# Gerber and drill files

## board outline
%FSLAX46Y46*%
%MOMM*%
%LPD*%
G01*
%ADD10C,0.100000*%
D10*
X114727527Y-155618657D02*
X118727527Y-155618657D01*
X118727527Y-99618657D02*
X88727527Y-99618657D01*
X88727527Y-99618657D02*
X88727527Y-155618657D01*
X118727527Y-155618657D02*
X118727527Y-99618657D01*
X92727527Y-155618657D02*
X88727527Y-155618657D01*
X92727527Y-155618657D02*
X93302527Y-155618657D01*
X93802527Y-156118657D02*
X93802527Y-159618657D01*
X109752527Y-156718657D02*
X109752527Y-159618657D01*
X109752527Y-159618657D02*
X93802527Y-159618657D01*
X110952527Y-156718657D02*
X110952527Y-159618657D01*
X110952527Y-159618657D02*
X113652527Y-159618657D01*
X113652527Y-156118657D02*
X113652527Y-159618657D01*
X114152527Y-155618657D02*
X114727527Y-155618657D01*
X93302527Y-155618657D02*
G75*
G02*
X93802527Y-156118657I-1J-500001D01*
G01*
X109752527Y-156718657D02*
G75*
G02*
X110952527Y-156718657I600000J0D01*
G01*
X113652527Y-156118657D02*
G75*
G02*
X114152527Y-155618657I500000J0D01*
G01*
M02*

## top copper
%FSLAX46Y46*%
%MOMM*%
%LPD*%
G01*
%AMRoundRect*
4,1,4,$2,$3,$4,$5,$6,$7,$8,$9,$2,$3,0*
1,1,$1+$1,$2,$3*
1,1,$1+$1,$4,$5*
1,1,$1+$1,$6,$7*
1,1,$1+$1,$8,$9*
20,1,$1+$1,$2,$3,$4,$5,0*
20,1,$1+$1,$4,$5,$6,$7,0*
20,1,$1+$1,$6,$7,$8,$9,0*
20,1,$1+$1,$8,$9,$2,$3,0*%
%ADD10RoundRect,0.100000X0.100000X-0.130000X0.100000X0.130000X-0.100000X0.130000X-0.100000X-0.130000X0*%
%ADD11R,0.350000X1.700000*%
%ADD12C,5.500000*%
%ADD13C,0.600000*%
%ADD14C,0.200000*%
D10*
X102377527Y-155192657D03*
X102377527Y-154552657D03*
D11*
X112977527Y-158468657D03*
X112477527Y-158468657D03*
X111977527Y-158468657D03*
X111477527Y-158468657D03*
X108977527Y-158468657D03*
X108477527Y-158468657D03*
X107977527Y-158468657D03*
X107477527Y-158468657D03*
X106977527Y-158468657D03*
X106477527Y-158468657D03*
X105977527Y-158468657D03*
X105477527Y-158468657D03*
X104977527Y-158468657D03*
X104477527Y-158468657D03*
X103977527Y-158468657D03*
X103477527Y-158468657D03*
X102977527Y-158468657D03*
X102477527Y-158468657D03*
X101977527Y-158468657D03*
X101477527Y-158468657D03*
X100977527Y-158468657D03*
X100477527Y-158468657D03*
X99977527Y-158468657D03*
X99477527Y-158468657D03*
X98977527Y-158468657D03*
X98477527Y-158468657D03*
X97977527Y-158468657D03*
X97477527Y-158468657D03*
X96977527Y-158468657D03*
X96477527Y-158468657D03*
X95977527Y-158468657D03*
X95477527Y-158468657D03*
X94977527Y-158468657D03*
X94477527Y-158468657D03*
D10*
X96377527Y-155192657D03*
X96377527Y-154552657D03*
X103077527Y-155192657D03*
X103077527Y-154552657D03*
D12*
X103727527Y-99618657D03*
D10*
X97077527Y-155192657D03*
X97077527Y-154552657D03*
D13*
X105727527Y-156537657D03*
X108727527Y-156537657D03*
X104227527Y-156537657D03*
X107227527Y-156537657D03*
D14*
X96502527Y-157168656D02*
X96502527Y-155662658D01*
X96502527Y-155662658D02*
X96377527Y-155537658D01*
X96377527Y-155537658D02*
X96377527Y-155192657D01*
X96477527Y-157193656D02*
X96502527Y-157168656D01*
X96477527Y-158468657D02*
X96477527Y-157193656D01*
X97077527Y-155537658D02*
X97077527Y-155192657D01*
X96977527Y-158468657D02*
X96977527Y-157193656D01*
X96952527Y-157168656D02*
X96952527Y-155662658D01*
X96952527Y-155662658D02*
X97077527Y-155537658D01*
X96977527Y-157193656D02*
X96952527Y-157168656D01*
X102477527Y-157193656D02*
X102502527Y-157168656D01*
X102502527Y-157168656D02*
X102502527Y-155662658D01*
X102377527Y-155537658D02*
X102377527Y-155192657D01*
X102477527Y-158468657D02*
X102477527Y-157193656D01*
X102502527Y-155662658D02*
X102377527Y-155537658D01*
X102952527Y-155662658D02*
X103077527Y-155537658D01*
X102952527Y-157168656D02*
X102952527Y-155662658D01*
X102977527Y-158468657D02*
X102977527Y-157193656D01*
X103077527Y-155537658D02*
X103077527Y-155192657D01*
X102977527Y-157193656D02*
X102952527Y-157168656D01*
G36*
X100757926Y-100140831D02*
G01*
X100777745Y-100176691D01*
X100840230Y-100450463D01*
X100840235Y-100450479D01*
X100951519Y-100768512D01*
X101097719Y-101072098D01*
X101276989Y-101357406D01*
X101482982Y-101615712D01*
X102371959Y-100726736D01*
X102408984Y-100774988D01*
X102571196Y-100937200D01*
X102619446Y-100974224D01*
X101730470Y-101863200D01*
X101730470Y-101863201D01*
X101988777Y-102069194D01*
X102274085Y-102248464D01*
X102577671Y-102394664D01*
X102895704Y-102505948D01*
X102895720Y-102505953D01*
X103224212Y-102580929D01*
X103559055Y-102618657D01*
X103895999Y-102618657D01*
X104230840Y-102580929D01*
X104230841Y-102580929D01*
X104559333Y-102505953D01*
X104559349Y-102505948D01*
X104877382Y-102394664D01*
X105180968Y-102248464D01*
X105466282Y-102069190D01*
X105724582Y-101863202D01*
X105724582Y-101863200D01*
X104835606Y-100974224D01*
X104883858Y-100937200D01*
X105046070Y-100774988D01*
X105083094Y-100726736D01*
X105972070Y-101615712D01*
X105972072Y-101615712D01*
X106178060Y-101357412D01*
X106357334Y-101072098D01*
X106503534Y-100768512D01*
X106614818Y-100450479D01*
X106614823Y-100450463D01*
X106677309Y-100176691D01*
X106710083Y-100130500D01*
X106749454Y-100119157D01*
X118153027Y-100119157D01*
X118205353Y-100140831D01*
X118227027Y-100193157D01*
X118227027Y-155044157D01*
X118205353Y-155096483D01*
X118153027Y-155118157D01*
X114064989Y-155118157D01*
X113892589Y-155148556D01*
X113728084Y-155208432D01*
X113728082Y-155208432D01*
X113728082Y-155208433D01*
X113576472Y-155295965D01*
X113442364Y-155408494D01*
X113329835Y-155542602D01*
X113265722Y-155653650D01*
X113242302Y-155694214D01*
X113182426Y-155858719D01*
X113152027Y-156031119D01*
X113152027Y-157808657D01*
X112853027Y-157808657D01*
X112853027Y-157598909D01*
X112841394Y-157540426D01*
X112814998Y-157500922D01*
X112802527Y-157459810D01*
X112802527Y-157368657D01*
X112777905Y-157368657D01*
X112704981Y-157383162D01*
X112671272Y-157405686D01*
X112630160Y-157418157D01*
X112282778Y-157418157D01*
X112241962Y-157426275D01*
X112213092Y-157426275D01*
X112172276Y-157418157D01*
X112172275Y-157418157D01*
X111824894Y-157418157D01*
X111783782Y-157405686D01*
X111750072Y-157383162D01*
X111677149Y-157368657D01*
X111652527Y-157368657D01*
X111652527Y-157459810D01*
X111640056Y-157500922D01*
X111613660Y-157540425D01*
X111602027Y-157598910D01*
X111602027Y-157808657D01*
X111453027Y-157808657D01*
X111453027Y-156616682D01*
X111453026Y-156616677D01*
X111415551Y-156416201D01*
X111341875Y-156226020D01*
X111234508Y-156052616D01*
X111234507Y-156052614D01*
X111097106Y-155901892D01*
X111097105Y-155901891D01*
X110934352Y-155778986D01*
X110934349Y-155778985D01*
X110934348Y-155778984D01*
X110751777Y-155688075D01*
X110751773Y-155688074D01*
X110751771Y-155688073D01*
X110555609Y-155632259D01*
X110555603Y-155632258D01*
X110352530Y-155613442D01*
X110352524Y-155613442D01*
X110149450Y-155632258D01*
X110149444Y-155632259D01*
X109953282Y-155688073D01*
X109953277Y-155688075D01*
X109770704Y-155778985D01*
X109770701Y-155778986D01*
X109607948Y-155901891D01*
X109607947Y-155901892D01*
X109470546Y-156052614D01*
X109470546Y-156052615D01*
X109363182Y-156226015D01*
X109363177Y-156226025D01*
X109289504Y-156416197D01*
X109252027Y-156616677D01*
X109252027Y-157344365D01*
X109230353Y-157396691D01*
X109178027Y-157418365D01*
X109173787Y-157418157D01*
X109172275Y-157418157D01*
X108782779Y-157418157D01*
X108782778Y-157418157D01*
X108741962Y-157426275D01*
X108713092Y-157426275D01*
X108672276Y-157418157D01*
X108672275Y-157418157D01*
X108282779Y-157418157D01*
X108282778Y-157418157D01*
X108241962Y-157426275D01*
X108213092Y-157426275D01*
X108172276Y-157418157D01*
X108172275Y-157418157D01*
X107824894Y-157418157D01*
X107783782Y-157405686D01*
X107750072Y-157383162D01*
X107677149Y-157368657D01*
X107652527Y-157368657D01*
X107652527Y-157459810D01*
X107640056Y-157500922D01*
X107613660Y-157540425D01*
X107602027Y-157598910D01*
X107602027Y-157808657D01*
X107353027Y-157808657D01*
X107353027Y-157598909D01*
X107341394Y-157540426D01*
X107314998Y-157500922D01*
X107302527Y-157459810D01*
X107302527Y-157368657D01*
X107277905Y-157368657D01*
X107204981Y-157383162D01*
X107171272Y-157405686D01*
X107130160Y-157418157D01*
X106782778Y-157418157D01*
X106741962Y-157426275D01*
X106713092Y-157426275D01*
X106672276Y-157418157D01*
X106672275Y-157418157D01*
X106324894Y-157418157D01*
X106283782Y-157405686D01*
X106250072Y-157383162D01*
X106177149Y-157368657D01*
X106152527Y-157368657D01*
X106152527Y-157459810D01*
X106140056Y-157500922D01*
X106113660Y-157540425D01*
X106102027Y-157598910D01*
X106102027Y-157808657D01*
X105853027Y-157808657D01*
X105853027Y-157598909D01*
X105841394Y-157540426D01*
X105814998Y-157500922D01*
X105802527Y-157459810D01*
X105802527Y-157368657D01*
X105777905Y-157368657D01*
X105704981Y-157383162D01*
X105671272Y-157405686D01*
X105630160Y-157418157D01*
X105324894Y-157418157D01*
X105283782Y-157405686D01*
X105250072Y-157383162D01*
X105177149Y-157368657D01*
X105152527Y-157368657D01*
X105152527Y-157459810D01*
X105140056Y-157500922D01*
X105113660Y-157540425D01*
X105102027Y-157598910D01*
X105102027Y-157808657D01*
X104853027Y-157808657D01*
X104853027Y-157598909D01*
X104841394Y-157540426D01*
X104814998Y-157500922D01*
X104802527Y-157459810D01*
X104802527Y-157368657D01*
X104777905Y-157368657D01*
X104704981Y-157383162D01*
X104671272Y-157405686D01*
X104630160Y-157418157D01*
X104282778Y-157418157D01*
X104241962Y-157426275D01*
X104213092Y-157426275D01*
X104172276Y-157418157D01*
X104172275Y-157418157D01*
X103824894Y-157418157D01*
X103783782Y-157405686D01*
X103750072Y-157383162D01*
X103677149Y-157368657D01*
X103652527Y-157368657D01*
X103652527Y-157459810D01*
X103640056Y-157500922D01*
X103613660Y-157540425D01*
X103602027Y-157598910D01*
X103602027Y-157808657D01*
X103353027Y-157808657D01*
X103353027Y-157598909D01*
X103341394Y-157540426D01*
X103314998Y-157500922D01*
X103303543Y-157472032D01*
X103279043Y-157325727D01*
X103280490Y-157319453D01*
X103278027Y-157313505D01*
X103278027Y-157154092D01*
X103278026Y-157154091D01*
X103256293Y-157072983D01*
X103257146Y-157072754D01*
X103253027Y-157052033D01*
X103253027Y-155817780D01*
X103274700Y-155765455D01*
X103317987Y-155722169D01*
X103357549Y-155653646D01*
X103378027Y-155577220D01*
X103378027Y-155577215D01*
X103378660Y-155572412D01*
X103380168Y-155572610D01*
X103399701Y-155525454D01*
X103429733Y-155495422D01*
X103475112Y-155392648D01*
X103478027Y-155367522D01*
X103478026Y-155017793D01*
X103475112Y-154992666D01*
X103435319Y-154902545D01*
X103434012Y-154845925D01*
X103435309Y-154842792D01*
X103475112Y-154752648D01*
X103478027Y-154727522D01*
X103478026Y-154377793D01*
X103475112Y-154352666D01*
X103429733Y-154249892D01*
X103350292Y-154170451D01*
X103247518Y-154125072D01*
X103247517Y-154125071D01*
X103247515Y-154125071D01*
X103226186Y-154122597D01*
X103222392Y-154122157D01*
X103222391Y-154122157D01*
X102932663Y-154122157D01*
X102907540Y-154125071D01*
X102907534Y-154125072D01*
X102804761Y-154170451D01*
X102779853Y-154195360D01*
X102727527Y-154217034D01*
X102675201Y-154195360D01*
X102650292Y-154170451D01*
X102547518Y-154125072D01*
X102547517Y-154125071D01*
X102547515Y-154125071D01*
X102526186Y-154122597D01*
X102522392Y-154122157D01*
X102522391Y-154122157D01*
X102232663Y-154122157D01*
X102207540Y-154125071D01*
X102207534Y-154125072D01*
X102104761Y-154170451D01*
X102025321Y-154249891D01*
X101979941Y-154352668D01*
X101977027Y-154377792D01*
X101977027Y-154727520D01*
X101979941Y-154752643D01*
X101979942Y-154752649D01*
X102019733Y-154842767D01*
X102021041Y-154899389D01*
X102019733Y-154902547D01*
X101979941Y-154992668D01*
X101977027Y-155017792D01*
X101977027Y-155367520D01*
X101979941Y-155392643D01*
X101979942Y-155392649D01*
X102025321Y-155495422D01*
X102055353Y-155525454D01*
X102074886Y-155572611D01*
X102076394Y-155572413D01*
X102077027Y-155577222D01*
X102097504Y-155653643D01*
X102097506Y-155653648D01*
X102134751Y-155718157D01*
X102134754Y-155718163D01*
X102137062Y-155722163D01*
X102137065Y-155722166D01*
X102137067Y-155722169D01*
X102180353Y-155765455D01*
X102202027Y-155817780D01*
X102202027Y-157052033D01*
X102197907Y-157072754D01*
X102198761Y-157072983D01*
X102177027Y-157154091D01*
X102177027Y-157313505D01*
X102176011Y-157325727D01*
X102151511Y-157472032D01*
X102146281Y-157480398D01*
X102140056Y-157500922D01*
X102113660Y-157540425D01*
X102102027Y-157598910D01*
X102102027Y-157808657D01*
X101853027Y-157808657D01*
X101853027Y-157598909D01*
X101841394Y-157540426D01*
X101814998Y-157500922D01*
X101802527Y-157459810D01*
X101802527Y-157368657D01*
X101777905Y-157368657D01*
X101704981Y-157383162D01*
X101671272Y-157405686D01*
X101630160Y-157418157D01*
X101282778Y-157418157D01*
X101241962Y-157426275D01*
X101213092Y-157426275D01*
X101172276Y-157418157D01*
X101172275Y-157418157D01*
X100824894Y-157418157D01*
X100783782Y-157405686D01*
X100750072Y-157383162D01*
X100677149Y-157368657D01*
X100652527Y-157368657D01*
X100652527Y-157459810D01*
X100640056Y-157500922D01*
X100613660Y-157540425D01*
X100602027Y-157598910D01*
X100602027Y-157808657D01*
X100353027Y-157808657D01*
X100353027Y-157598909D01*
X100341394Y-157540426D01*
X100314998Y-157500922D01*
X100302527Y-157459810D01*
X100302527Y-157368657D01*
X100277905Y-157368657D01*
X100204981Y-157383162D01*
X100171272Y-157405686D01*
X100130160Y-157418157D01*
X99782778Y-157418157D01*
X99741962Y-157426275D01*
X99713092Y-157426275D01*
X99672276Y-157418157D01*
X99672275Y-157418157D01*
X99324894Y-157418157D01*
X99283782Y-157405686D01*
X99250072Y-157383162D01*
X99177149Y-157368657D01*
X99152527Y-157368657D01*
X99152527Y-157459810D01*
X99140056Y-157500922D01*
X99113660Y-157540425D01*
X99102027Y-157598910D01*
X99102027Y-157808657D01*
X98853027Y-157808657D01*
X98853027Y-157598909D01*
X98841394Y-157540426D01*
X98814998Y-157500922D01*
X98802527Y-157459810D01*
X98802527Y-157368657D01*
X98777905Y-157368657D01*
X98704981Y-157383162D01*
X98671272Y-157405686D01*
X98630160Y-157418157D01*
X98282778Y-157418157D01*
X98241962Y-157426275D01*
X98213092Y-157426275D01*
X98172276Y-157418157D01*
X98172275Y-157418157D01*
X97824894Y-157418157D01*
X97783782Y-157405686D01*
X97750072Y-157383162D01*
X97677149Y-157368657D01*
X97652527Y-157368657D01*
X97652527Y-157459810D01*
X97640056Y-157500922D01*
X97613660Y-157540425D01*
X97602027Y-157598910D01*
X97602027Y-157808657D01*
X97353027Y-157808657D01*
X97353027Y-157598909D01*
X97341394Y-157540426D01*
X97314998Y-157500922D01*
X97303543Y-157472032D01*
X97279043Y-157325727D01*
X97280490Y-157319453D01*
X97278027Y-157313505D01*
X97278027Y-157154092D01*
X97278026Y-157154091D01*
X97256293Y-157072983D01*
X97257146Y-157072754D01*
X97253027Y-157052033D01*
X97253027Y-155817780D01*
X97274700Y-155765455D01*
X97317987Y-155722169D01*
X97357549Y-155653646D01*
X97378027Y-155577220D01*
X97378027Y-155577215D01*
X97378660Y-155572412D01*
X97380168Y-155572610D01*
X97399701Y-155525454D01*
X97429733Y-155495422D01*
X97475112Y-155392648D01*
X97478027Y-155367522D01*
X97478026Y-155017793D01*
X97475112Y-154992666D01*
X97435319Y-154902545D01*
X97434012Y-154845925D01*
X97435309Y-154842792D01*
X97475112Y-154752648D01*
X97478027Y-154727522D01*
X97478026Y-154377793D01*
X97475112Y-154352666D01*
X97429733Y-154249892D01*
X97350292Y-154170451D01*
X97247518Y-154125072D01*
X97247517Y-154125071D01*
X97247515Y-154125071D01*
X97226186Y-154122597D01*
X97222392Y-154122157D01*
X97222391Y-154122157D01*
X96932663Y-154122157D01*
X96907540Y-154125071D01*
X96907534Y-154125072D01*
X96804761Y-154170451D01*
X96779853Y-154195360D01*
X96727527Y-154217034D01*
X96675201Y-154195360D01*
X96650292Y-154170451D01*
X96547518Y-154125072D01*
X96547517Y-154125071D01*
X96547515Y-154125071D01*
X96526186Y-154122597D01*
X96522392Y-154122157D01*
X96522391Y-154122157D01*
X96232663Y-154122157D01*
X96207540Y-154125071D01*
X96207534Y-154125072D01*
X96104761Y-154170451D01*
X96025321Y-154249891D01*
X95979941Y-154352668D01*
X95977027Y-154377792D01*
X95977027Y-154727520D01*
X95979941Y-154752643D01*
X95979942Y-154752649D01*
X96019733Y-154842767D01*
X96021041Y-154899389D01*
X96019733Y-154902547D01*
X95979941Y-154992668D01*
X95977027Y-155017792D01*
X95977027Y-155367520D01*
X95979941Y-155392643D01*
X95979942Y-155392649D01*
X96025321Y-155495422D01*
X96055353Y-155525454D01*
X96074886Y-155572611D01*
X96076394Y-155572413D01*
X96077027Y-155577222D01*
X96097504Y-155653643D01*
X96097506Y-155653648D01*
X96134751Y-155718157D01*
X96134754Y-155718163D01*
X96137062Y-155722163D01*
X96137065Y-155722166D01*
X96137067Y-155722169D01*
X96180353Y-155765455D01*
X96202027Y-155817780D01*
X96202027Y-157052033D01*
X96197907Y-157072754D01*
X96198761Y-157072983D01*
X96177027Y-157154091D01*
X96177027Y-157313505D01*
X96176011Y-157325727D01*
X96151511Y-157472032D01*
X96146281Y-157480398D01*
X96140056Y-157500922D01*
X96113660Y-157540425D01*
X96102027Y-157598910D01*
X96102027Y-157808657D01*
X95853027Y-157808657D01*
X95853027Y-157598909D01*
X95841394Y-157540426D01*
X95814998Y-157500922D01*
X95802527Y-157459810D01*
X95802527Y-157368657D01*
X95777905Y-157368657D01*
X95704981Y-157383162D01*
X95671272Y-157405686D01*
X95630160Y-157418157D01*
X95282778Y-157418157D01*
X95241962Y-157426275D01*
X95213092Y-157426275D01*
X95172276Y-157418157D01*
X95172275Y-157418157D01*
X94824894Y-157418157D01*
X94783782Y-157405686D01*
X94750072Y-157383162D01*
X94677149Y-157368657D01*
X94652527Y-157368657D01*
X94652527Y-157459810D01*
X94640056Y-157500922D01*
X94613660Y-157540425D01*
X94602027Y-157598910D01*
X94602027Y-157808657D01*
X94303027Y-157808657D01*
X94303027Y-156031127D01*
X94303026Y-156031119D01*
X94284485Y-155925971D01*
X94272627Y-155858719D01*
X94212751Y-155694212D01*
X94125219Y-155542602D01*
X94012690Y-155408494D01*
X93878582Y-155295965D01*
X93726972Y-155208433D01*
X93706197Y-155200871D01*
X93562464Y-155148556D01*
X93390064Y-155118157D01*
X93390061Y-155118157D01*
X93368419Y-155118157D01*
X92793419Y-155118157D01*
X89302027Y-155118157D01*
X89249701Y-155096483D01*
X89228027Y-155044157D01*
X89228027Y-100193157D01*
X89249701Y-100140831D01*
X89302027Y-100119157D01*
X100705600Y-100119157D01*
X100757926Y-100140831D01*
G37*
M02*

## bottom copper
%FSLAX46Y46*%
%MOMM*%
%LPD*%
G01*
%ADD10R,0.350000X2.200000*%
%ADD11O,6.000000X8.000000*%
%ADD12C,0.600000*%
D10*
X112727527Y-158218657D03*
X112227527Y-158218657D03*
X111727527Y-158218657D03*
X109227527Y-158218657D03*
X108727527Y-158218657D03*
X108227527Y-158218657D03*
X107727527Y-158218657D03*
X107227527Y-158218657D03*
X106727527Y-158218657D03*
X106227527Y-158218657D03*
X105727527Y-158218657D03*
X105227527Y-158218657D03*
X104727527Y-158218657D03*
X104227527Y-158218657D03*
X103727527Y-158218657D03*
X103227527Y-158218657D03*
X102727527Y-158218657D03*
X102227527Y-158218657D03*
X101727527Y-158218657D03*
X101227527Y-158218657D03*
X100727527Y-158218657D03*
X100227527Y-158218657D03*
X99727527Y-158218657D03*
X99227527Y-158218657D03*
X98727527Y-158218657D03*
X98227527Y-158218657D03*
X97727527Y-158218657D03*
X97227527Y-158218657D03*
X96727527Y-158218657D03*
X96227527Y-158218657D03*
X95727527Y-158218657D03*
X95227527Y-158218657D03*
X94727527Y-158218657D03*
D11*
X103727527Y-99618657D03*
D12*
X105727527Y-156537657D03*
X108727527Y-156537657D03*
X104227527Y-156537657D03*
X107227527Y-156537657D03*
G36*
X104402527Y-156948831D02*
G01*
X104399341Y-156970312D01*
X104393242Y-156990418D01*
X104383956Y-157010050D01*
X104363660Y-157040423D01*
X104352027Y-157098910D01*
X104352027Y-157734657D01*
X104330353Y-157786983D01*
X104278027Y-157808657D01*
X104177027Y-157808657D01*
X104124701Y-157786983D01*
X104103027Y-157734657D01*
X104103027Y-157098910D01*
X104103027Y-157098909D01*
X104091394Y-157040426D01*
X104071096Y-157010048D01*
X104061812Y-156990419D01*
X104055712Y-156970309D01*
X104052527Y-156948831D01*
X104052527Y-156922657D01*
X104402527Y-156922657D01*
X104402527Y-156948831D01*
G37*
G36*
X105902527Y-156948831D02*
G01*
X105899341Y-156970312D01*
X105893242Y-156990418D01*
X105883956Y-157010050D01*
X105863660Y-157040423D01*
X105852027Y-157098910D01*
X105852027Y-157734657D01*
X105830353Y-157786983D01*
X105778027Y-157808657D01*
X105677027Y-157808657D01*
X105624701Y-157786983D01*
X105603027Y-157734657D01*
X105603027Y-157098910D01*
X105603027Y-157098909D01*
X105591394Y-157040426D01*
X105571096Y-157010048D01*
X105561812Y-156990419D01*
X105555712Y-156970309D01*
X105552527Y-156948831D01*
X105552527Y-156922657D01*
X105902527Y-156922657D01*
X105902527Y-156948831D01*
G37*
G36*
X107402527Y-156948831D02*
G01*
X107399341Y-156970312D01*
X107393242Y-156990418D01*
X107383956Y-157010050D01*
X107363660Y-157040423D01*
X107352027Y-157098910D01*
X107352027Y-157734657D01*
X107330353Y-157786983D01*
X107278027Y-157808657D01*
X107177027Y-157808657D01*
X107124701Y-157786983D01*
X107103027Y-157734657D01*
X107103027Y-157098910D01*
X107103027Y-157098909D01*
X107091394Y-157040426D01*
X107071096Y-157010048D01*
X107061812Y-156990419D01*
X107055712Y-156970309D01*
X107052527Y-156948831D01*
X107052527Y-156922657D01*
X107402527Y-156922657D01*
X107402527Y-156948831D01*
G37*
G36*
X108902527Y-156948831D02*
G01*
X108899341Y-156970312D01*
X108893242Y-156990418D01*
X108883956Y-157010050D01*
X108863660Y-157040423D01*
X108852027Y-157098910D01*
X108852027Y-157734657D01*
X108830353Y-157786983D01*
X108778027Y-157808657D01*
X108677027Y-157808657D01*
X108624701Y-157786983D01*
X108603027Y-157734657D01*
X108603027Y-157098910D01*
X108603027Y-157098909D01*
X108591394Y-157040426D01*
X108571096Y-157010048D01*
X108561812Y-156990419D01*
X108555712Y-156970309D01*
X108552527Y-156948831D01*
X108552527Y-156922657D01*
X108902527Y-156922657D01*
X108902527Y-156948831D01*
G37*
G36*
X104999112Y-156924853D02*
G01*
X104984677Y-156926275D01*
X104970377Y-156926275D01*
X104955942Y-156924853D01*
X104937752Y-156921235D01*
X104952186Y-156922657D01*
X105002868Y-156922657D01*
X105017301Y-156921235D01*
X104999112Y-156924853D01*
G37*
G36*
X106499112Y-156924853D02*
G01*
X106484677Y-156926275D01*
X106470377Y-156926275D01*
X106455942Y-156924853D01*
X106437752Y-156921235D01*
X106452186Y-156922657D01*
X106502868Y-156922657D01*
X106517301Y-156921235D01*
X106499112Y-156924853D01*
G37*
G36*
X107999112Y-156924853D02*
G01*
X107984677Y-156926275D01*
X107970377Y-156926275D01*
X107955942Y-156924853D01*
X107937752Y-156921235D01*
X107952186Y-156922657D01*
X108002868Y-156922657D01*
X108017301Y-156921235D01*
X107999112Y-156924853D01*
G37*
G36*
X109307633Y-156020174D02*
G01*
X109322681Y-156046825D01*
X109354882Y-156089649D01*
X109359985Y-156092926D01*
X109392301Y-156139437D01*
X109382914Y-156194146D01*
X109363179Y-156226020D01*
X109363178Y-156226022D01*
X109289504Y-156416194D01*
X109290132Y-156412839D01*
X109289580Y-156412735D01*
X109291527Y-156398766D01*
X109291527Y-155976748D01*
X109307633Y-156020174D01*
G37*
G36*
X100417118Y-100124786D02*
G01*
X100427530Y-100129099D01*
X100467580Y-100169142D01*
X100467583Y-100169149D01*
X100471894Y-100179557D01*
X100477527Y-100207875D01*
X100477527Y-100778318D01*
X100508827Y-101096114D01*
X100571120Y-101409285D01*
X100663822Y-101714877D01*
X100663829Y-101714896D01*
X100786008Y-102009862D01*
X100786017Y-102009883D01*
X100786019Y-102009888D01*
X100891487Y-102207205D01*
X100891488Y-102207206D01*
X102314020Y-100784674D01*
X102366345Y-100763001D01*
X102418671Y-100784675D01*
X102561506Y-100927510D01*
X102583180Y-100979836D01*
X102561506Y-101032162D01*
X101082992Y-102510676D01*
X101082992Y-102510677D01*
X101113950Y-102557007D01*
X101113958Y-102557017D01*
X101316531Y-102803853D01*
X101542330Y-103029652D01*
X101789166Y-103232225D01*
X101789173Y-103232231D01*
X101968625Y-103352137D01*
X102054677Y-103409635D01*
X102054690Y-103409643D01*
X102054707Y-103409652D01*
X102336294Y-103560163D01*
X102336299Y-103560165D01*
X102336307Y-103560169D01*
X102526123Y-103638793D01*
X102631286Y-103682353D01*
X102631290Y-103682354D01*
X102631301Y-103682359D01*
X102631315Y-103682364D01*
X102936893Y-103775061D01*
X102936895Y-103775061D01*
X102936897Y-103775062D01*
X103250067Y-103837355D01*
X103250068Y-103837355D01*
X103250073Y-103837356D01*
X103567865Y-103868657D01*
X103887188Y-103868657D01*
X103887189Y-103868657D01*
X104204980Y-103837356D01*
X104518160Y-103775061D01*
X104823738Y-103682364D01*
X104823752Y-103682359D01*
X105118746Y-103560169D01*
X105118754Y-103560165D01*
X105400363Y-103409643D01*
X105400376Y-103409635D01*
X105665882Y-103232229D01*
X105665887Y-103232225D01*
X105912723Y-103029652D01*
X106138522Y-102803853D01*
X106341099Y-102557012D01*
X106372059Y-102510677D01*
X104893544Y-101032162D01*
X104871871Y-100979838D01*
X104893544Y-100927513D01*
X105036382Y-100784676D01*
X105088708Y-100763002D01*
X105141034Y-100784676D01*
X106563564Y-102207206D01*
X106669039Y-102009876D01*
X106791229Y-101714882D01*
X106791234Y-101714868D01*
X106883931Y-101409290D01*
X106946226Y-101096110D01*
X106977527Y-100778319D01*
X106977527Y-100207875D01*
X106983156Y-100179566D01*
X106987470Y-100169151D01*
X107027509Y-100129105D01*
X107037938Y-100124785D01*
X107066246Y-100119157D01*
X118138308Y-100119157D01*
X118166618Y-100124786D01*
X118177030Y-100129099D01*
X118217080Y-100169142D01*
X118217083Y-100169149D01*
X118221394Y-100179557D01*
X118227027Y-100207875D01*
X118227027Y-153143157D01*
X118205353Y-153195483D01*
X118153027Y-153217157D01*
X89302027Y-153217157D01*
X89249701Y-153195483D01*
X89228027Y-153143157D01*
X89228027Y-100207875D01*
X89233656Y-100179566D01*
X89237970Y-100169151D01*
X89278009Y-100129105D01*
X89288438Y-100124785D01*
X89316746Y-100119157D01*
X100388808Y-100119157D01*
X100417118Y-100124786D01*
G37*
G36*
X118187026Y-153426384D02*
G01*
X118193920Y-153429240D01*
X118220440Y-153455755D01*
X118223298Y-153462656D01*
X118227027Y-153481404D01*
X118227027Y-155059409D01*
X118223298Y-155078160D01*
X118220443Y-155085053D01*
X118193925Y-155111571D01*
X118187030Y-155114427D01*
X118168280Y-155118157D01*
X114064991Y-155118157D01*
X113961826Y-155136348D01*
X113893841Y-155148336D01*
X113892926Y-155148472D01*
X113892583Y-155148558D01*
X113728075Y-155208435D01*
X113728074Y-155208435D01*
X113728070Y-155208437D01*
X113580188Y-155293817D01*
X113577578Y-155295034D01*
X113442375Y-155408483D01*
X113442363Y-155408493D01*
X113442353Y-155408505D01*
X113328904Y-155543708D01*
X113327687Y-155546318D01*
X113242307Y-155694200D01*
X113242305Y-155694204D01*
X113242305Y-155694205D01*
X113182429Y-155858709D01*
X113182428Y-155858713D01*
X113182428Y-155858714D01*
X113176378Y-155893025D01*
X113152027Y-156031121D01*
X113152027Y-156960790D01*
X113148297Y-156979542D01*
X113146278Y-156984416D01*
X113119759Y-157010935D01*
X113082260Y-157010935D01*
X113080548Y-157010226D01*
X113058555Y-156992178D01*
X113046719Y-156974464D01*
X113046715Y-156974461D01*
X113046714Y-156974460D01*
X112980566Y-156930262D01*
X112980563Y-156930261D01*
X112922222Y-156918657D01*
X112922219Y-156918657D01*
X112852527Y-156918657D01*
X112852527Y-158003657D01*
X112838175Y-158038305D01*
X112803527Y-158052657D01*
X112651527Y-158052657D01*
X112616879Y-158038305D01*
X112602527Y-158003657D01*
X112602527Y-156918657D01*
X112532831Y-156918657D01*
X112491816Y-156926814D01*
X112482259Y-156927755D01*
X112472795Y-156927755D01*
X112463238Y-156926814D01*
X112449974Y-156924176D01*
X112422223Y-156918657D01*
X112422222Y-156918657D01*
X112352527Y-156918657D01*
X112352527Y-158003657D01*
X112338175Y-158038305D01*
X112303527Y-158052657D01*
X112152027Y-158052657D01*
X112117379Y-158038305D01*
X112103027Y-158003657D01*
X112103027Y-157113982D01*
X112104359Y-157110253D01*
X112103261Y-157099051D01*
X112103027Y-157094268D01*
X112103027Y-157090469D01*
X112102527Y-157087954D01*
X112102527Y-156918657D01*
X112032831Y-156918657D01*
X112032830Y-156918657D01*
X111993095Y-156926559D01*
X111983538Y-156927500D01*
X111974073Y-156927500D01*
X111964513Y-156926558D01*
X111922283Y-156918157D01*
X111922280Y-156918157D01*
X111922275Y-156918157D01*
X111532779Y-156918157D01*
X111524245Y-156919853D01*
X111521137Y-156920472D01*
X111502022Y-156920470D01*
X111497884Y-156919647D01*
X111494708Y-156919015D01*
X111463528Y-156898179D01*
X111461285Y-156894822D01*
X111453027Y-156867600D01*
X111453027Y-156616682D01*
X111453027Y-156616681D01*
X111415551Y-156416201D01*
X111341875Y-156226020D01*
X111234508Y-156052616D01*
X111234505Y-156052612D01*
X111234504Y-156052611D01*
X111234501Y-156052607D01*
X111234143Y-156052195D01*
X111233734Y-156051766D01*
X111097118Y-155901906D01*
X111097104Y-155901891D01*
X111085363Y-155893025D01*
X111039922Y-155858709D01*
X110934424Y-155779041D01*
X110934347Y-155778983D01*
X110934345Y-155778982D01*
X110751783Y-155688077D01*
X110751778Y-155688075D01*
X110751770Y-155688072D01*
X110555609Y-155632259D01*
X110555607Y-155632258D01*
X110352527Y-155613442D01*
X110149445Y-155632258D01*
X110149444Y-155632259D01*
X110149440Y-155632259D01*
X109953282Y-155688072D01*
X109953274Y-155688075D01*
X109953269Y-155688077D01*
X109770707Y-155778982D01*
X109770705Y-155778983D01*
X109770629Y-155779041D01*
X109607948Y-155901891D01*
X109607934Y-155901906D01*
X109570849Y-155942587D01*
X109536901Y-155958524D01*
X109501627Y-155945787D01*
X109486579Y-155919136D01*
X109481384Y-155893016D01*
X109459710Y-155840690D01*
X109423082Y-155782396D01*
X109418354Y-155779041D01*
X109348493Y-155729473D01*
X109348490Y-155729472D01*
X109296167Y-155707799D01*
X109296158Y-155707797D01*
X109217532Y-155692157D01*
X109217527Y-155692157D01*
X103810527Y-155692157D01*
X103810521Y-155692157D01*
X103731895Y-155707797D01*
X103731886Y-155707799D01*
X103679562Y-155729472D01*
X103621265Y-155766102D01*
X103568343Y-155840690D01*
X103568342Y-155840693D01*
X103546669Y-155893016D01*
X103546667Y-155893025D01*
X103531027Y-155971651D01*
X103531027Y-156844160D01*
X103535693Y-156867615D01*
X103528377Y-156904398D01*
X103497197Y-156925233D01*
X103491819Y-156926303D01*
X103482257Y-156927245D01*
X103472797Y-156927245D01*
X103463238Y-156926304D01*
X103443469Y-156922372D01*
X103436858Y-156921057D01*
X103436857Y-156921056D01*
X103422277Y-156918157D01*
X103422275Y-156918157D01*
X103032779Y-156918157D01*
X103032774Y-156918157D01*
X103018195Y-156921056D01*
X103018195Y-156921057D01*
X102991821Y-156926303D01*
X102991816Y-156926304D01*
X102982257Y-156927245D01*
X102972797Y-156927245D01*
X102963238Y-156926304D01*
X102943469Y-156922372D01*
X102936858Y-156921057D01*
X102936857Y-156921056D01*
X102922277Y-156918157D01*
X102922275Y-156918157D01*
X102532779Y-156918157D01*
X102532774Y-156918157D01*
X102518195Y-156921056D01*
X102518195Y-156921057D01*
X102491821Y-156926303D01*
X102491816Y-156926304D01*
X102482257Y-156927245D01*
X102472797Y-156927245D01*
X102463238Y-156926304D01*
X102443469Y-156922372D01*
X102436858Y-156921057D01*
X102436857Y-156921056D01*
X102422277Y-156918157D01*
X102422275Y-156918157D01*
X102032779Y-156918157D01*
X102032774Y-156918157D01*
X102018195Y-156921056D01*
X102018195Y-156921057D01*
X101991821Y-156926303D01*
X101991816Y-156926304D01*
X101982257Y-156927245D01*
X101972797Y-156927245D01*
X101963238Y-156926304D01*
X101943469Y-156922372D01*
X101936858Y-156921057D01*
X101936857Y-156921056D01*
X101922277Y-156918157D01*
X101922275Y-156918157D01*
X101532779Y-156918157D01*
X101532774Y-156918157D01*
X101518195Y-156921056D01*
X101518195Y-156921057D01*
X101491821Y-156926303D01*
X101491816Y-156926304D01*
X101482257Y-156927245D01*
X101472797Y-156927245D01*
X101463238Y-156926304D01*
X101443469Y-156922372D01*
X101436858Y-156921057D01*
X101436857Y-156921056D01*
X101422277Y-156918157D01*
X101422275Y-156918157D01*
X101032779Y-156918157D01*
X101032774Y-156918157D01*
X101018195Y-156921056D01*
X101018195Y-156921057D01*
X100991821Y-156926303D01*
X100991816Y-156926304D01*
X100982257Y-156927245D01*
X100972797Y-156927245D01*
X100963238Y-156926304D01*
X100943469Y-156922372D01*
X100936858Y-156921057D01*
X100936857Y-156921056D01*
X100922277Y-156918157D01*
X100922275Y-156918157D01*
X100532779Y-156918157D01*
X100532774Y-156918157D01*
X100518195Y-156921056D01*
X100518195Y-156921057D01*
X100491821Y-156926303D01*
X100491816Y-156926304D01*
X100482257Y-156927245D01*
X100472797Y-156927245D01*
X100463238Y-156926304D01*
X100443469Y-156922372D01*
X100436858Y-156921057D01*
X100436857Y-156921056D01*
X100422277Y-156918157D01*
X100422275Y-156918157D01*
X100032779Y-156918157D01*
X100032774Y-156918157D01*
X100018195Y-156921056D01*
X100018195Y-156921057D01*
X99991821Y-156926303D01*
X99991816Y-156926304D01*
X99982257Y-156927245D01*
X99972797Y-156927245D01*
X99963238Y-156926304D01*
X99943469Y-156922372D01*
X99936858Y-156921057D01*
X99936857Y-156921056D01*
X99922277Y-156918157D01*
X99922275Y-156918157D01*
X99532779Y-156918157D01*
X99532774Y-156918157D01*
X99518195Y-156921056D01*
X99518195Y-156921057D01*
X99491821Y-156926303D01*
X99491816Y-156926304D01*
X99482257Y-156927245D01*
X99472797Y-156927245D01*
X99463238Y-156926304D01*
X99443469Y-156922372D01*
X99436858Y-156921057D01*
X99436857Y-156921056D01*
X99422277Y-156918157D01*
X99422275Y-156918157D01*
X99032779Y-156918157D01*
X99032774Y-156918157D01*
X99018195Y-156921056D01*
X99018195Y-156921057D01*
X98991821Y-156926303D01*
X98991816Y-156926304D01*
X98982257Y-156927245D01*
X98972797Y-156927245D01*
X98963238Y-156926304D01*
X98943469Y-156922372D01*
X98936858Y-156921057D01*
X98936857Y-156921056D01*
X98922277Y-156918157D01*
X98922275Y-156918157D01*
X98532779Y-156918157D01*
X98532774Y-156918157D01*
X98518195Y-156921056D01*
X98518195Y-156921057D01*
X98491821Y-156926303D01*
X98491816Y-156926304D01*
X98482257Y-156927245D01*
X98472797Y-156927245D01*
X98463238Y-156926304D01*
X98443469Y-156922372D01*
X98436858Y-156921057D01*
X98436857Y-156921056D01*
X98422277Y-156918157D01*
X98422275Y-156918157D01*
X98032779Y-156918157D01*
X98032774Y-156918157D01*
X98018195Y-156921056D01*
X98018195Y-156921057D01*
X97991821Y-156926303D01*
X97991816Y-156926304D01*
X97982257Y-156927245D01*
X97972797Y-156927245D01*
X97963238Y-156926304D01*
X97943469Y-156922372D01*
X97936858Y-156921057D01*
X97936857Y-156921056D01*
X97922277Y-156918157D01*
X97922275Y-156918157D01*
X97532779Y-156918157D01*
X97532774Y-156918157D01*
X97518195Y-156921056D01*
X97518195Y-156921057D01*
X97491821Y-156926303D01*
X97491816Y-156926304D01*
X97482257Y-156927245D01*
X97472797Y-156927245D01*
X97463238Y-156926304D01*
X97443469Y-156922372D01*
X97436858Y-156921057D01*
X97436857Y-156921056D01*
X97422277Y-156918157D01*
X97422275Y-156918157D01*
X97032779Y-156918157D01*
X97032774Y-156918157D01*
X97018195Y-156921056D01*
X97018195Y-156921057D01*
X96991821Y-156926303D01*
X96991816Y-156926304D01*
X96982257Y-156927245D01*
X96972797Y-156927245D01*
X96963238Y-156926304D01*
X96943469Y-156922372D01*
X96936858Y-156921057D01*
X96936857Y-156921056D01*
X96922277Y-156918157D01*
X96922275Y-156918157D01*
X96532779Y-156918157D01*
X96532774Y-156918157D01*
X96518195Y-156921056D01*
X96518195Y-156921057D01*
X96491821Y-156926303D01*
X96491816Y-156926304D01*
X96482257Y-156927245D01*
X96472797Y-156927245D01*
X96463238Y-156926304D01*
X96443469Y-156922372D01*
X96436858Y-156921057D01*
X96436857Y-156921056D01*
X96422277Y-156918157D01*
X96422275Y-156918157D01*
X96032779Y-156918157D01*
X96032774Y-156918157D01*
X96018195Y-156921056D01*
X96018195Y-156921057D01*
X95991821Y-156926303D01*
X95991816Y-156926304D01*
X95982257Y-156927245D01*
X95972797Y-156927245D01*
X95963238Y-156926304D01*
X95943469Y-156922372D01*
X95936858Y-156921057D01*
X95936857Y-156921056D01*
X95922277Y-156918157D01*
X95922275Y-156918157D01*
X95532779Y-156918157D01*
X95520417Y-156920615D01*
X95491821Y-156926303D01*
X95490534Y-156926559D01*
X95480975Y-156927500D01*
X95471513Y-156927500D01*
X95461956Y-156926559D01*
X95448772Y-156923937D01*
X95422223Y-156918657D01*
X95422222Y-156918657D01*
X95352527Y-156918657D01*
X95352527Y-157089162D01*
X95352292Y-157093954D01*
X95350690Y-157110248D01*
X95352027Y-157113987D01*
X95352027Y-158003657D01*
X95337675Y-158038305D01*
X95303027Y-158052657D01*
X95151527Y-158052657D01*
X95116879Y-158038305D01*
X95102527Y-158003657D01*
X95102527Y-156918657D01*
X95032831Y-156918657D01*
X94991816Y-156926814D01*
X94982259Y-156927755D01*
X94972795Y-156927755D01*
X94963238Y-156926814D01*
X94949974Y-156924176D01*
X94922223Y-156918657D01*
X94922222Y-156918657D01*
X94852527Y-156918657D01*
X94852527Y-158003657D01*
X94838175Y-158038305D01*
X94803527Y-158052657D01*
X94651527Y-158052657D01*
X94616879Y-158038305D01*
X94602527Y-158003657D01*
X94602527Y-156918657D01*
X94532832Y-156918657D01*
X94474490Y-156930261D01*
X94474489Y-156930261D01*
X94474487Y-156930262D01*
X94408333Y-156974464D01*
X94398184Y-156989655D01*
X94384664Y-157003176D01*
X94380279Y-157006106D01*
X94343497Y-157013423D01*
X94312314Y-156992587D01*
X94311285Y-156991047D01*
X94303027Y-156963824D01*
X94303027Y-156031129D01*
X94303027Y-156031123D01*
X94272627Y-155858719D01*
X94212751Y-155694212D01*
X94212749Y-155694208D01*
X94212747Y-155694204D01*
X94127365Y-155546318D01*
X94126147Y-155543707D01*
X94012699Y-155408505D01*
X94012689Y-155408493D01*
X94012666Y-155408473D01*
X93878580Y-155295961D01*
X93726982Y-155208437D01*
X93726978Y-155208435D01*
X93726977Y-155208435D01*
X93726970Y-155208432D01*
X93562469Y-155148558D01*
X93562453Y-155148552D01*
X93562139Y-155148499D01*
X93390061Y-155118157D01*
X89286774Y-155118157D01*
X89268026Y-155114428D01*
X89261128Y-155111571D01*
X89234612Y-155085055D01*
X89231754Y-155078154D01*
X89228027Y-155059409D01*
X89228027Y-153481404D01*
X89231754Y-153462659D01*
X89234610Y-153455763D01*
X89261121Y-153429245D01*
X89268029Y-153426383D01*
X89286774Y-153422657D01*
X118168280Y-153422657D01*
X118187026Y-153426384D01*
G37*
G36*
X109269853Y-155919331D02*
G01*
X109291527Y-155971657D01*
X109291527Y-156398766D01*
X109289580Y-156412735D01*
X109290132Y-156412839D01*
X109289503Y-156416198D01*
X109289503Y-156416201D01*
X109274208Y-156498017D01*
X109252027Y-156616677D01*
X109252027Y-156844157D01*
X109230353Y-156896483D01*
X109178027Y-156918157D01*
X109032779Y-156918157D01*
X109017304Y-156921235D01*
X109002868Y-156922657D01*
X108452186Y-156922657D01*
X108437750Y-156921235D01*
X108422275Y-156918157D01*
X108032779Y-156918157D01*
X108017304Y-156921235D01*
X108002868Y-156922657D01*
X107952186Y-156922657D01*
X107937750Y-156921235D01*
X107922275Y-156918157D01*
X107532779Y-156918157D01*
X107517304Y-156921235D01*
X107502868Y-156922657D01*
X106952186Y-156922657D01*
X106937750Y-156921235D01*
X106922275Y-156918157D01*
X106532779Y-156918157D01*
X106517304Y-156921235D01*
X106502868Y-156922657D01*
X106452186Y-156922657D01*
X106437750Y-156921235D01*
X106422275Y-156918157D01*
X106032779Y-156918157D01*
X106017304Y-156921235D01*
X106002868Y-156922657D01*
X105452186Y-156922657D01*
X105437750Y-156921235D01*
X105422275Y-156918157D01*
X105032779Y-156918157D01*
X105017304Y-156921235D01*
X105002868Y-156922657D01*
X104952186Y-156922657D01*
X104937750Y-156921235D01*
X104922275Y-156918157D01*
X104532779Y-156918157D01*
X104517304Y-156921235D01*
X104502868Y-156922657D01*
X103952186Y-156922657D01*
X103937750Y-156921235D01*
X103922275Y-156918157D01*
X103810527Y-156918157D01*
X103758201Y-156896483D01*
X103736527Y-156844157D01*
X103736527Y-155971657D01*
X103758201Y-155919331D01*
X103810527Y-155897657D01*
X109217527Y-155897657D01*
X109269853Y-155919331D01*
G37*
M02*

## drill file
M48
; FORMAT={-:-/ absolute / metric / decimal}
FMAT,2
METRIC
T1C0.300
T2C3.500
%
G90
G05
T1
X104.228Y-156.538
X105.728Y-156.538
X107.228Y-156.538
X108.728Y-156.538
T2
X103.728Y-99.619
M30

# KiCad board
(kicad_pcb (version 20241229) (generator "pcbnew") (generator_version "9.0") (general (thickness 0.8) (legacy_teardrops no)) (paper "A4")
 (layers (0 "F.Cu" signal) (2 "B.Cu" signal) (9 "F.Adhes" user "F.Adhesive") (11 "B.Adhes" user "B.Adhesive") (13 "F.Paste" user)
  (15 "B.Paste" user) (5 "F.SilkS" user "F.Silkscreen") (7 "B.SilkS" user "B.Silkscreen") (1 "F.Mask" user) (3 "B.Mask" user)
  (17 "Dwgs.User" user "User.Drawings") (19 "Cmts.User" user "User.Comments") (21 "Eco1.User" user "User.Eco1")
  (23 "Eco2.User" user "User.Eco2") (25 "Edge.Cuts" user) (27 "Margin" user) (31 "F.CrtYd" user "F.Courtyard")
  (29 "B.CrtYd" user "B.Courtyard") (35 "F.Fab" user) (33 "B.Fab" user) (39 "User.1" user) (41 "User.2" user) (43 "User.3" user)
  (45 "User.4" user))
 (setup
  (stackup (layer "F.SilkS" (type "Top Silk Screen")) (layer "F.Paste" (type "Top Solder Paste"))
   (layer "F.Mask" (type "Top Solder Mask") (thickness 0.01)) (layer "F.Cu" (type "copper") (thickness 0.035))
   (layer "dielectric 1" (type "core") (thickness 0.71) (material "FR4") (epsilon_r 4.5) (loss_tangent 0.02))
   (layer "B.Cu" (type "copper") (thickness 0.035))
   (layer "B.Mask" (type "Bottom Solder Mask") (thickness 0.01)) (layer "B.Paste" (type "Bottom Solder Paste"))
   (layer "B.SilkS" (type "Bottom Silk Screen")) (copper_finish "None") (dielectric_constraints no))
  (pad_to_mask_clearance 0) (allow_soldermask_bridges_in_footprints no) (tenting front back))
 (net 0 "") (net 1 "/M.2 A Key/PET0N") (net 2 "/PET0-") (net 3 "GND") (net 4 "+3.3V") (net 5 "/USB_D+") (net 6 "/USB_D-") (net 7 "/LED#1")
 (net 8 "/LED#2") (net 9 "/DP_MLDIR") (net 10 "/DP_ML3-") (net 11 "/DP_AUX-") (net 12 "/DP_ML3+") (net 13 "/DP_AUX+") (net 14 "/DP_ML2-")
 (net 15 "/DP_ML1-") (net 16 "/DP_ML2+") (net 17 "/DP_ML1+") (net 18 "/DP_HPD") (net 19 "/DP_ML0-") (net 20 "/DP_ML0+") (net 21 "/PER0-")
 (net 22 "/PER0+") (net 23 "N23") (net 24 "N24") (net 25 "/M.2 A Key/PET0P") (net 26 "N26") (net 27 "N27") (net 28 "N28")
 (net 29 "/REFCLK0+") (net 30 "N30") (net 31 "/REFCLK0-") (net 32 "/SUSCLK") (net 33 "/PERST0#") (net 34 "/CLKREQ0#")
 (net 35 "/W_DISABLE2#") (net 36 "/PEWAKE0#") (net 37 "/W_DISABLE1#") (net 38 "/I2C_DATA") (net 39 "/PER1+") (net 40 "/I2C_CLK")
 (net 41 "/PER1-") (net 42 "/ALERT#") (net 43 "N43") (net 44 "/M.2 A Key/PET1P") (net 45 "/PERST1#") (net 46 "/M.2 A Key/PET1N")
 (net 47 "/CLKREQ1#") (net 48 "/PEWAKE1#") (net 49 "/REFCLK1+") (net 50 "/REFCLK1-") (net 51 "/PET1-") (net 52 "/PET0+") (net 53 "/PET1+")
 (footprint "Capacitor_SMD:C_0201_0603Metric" (layer "F.Cu") (at 102.377527 154.872657 90)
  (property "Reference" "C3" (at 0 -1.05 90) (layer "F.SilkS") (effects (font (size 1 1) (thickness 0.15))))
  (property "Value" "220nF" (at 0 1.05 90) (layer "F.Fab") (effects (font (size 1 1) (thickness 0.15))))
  (pad "" smd roundrect (at -0.345 0 90) (size 0.318 0.36) (layers "F.Paste") (roundrect_rratio 0.25))
  (pad "" smd roundrect (at 0.345 0 90) (size 0.318 0.36) (layers "F.Paste") (roundrect_rratio 0.25))
  (pad "1" smd roundrect (at -0.32 0 90) (size 0.46 0.4) (layers "F.Cu" "F.Mask") (roundrect_rratio 0.25) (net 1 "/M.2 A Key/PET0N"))
  (pad "2" smd roundrect (at 0.32 0 90) (size 0.46 0.4) (layers "F.Cu" "F.Mask") (roundrect_rratio 0.25) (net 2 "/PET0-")))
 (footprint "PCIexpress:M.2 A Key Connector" (layer "F.Cu") (at 103.727527 158.508657)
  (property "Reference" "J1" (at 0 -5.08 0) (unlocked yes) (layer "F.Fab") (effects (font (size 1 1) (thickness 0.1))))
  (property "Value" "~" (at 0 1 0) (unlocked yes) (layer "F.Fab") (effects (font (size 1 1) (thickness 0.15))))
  (fp_line (start -11 -2.89) (end -10.425 -2.89) (stroke (width 0.1) (type default)) (layer "Edge.Cuts"))
  (fp_line (start -9.925 -2.39) (end -9.925 1.11) (stroke (width 0.1) (type default)) (layer "Edge.Cuts"))
  (fp_line (start 6.025 -1.79) (end 6.025 1.11) (stroke (width 0.1) (type default)) (layer "Edge.Cuts"))
  (fp_line (start 6.025 1.11) (end -9.925 1.11) (stroke (width 0.1) (type default)) (layer "Edge.Cuts"))
  (fp_line (start 7.225 -1.79) (end 7.225 1.11) (stroke (width 0.1) (type default)) (layer "Edge.Cuts"))
  (fp_line (start 7.225 1.11) (end 9.925 1.11) (stroke (width 0.1) (type default)) (layer "Edge.Cuts"))
  (fp_line (start 9.925 -2.39) (end 9.925 1.11) (stroke (width 0.1) (type default)) (layer "Edge.Cuts"))
  (fp_line (start 10.425 -2.89) (end 11 -2.89) (stroke (width 0.1) (type default)) (layer "Edge.Cuts"))
  (fp_arc (start -10.425 -2.89) (mid -10.071447 -2.743553) (end -9.925 -2.39) (stroke (width 0.1) (type default)) (layer "Edge.Cuts"))
  (fp_arc (start 6.025 -1.79) (mid 6.625 -2.39) (end 7.225 -1.79) (stroke (width 0.1) (type default)) (layer "Edge.Cuts"))
  (fp_arc (start 9.925 -2.39) (mid 10.071447 -2.743553) (end 10.425 -2.89) (stroke (width 0.1) (type default)) (layer "Edge.Cuts"))
  (pad "1" smd rect (at 9.25 -0.04 180) (size 0.35 1.7) (layers "F.Cu") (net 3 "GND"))
  (pad "2" smd rect (at 9 -0.29 180) (size 0.35 2.2) (layers "B.Cu") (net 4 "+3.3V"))
  (pad "3" smd rect (at 8.75 -0.04 180) (size 0.35 1.7) (layers "F.Cu") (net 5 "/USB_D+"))
  (pad "4" smd rect (at 8.5 -0.29 180) (size 0.35 2.2) (layers "B.Cu") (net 4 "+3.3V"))
  (pad "5" smd rect (at 8.25 -0.04 180) (size 0.35 1.7) (layers "F.Cu") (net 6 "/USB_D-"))
  (pad "6" smd rect (at 8 -0.29 180) (size 0.35 2.2) (layers "B.Cu") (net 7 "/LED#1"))
  (pad "7" smd rect (at 7.75 -0.04 180) (size 0.35 1.7) (layers "F.Cu") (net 3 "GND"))
  (pad "16" smd rect (at 5.5 -0.29 180) (size 0.35 2.2) (layers "B.Cu") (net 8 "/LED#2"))
  (pad "17" smd rect (at 5.25 -0.04 180) (size 0.35 1.7) (layers "F.Cu") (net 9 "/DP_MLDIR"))
  (pad "18" smd rect (at 5 -0.29 180) (size 0.35 2.2) (layers "B.Cu") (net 3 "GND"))
  (pad "19" smd rect (at 4.75 -0.04 180) (size 0.35 1.7) (layers "F.Cu") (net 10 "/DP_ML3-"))
  (pad "20" smd rect (at 4.5 -0.29 180) (size 0.35 2.2) (layers "B.Cu") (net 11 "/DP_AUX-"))
  (pad "21" smd rect (at 4.25 -0.04 180) (size 0.35 1.7) (layers "F.Cu") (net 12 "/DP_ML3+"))
  (pad "22" smd rect (at 4 -0.29 180) (size 0.35 2.2) (layers "B.Cu") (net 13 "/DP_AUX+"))
  (pad "23" smd rect (at 3.75 -0.04 180) (size 0.35 1.7) (layers "F.Cu") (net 3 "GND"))
  (pad "24" smd rect (at 3.5 -0.29 180) (size 0.35 2.2) (layers "B.Cu") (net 3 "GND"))
  (pad "25" smd rect (at 3.25 -0.04 180) (size 0.35 1.7) (layers "F.Cu") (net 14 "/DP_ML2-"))
  (pad "26" smd rect (at 3 -0.29 180) (size 0.35 2.2) (layers "B.Cu") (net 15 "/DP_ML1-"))
  (pad "27" smd rect (at 2.75 -0.04 180) (size 0.35 1.7) (layers "F.Cu") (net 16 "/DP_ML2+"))
  (pad "28" smd rect (at 2.5 -0.29 180) (size 0.35 2.2) (layers "B.Cu") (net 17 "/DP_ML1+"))
  (pad "29" smd rect (at 2.25 -0.04 180) (size 0.35 1.7) (layers "F.Cu") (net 3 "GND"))
  (pad "30" smd rect (at 2 -0.29 180) (size 0.35 2.2) (layers "B.Cu") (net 3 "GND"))
  (pad "31" smd rect (at 1.75 -0.04 180) (size 0.35 1.7) (layers "F.Cu") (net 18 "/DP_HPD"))
  (pad "32" smd rect (at 1.5 -0.29 180) (size 0.35 2.2) (layers "B.Cu") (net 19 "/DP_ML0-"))
  (pad "33" smd rect (at 1.25 -0.04 180) (size 0.35 1.7) (layers "F.Cu") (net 3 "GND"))
  (pad "34" smd rect (at 1 -0.29 180) (size 0.35 2.2) (layers "B.Cu") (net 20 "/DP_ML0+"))
  (pad "35" smd rect (at 0.75 -0.04 180) (size 0.35 1.7) (layers "F.Cu") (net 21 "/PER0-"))
  (pad "36" smd rect (at 0.5 -0.29 180) (size 0.35 2.2) (layers "B.Cu") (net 3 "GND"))
  (pad "37" smd rect (at 0.25 -0.04 180) (size 0.35 1.7) (layers "F.Cu") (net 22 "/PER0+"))
  (pad "38" smd rect (at 0 -0.29 180) (size 0.35 2.2) (layers "B.Cu") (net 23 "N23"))
  (pad "39" smd rect (at -0.25 -0.04 180) (size 0.35 1.7) (layers "F.Cu") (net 3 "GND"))
  (pad "40" smd rect (at -0.5 -0.29 180) (size 0.35 2.2) (layers "B.Cu") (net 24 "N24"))
  (pad "41" smd rect (at -0.75 -0.04 180) (size 0.35 1.7) (layers "F.Cu") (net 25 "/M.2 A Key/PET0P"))
  (pad "42" smd rect (at -1 -0.29 180) (size 0.35 2.2) (layers "B.Cu") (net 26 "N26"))
  (pad "43" smd rect (at -1.25 -0.04 180) (size 0.35 1.7) (layers "F.Cu") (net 1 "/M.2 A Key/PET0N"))
  (pad "44" smd rect (at -1.5 -0.29 180) (size 0.35 2.2) (layers "B.Cu") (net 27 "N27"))
  (pad "45" smd rect (at -1.75 -0.04 180) (size 0.35 1.7) (layers "F.Cu") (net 3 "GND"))
  (pad "46" smd rect (at -2 -0.29 180) (size 0.35 2.2) (layers "B.Cu") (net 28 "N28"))
  (pad "47" smd rect (at -2.25 -0.04 180) (size 0.35 1.7) (layers "F.Cu") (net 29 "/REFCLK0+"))
  (pad "48" smd rect (at -2.5 -0.29 180) (size 0.35 2.2) (layers "B.Cu") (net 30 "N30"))
  (pad "49" smd rect (at -2.75 -0.04 180) (size 0.35 1.7) (layers "F.Cu") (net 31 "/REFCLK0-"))
  (pad "50" smd rect (at -3 -0.29 180) (size 0.35 2.2) (layers "B.Cu") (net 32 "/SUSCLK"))
  (pad "51" smd rect (at -3.25 -0.04 180) (size 0.35 1.7) (layers "F.Cu") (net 3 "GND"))
  (pad "52" smd rect (at -3.5 -0.29 180) (size 0.35 2.2) (layers "B.Cu") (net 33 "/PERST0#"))
  (pad "53" smd rect (at -3.75 -0.04 180) (size 0.35 1.7) (layers "F.Cu") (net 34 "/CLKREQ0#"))
  (pad "54" smd rect (at -4 -0.29 180) (size 0.35 2.2) (layers "B.Cu") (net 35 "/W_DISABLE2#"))
  (pad "55" smd rect (at -4.25 -0.04 180) (size 0.35 1.7) (layers "F.Cu") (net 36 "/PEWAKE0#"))
  (pad "56" smd rect (at -4.5 -0.29 180) (size 0.35 2.2) (layers "B.Cu") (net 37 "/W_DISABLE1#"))
  (pad "57" smd rect (at -4.75 -0.04 180) (size 0.35 1.7) (layers "F.Cu") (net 3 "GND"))
  (pad "58" smd rect (at -5 -0.29 180) (size 0.35 2.2) (layers "B.Cu") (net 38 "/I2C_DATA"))
  (pad "59" smd rect (at -5.25 -0.04 180) (size 0.35 1.7) (layers "F.Cu") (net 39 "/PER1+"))
  (pad "60" smd rect (at -5.5 -0.29 180) (size 0.35 2.2) (layers "B.Cu") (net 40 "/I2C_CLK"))
  (pad "61" smd rect (at -5.75 -0.04 180) (size 0.35 1.7) (layers "F.Cu") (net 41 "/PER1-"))
  (pad "62" smd rect (at -6 -0.29 180) (size 0.35 2.2) (layers "B.Cu") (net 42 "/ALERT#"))
  (pad "63" smd rect (at -6.25 -0.04 180) (size 0.35 1.7) (layers "F.Cu") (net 3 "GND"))
  (pad "64" smd rect (at -6.5 -0.29 180) (size 0.35 2.2) (layers "B.Cu") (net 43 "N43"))
  (pad "65" smd rect (at -6.75 -0.04 180) (size 0.35 1.7) (layers "F.Cu") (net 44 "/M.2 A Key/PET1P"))
  (pad "66" smd rect (at -7 -0.29 180) (size 0.35 2.2) (layers "B.Cu") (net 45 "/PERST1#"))
  (pad "67" smd rect (at -7.25 -0.04 180) (size 0.35 1.7) (layers "F.Cu") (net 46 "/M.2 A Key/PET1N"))
  (pad "68" smd rect (at -7.5 -0.29 180) (size 0.35 2.2) (layers "B.Cu") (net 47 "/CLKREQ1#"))
  (pad "69" smd rect (at -7.75 -0.04 180) (size 0.35 1.7) (layers "F.Cu") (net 3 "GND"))
  (pad "70" smd rect (at -8 -0.29 180) (size 0.35 2.2) (layers "B.Cu") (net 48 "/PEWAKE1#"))
  (pad "71" smd rect (at -8.25 -0.04 180) (size 0.35 1.7) (layers "F.Cu") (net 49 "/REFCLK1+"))
  (pad "72" smd rect (at -8.5 -0.29 180) (size 0.35 2.2) (layers "B.Cu") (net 4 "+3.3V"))
  (pad "73" smd rect (at -8.75 -0.04 180) (size 0.35 1.7) (layers "F.Cu") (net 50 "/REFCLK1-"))
  (pad "74" smd rect (at -9 -0.29 180) (size 0.35 2.2) (layers "B.Cu") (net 4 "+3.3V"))
  (pad "75" smd rect (at -9.25 -0.04 180) (size 0.35 1.7) (layers "F.Cu") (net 3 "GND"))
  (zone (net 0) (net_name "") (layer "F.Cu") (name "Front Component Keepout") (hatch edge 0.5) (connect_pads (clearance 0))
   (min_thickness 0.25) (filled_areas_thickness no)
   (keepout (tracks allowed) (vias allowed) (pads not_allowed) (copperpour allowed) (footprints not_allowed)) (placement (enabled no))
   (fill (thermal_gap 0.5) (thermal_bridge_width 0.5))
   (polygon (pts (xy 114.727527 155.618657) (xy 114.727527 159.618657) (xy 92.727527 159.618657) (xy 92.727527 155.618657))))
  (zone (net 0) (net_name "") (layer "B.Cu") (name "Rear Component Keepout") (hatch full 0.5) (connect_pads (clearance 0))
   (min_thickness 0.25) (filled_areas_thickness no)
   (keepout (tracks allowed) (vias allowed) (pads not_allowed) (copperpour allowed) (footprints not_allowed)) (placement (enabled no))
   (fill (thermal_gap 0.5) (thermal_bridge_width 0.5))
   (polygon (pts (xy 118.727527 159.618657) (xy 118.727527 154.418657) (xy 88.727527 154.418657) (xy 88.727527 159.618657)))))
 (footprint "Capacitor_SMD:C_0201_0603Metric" (layer "F.Cu") (at 96.377527 154.872657 90)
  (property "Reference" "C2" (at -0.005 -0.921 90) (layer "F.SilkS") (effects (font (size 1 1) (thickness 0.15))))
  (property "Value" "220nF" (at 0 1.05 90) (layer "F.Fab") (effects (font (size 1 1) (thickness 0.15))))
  (pad "" smd roundrect (at -0.345 0 90) (size 0.318 0.36) (layers "F.Paste") (roundrect_rratio 0.25))
  (pad "" smd roundrect (at 0.345 0 90) (size 0.318 0.36) (layers "F.Paste") (roundrect_rratio 0.25))
  (pad "1" smd roundrect (at -0.32 0 90) (size 0.46 0.4) (layers "F.Cu" "F.Mask") (roundrect_rratio 0.25) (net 46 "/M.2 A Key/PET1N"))
  (pad "2" smd roundrect (at 0.32 0 90) (size 0.46 0.4) (layers "F.Cu" "F.Mask") (roundrect_rratio 0.25) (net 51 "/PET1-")))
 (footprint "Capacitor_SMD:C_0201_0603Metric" (layer "F.Cu") (at 103.077527 154.872657 90)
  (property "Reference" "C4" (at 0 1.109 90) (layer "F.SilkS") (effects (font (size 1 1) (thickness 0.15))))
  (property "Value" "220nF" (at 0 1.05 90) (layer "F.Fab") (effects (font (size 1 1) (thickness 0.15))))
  (pad "" smd roundrect (at -0.345 0 90) (size 0.318 0.36) (layers "F.Paste") (roundrect_rratio 0.25))
  (pad "" smd roundrect (at 0.345 0 90) (size 0.318 0.36) (layers "F.Paste") (roundrect_rratio 0.25))
  (pad "1" smd roundrect (at -0.32 0 90) (size 0.46 0.4) (layers "F.Cu" "F.Mask") (roundrect_rratio 0.25) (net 25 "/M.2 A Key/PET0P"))
  (pad "2" smd roundrect (at 0.32 0 90) (size 0.46 0.4) (layers "F.Cu" "F.Mask") (roundrect_rratio 0.25) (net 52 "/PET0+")))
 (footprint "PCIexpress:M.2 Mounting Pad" (layer "F.Cu") (at 103.727527 129.618657)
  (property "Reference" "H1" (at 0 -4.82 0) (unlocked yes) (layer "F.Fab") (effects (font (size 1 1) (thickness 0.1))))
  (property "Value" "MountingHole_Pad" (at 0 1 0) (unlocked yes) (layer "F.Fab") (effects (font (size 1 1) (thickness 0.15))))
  (pad "1" thru_hole circle (at 0 -30) (size 5.5 5.5) (drill 3.5) (layers "*.Cu" "*.Mask") (remove_unused_layers no) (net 3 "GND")
   (padstack (mode front_inner_back)
    (layer "Inner" (shape circle) (size 5.5 5.5) (zone_connect -1))
    (layer "B.Cu" (shape oval) (size 6 8) (thermal_bridge_angle 45) (zone_connect -1)))))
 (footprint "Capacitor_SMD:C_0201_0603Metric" (layer "F.Cu") (at 97.077527 154.872657 90)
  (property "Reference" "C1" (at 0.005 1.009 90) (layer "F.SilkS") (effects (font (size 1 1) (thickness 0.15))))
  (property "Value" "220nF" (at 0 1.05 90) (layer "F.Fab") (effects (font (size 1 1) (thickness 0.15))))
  (pad "" smd roundrect (at -0.345 0 90) (size 0.318 0.36) (layers "F.Paste") (roundrect_rratio 0.25))
  (pad "" smd roundrect (at 0.345 0 90) (size 0.318 0.36) (layers "F.Paste") (roundrect_rratio 0.25))
  (pad "1" smd roundrect (at -0.32 0 90) (size 0.46 0.4) (layers "F.Cu" "F.Mask") (roundrect_rratio 0.25) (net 44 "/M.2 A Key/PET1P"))
  (pad "2" smd roundrect (at 0.32 0 90) (size 0.46 0.4) (layers "F.Cu" "F.Mask") (roundrect_rratio 0.25) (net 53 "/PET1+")))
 (gr_line (start 114.727527 155.618657) (end 118.727527 155.618657) (stroke (width 0.1) (type default)) (layer "Edge.Cuts"))
 (gr_line (start 118.727527 99.618657) (end 88.727527 99.618657) (stroke (width 0.1) (type solid)) (layer "Edge.Cuts"))
 (gr_line (start 88.727527 99.618657) (end 88.727527 155.618657) (stroke (width 0.1) (type default)) (layer "Edge.Cuts"))
 (gr_line (start 118.727527 155.618657) (end 118.727527 99.618657) (stroke (width 0.1) (type default)) (layer "Edge.Cuts"))
 (gr_line (start 92.727527 155.618657) (end 88.727527 155.618657) (stroke (width 0.1) (type default)) (layer "Edge.Cuts"))
 (via (at 105.727527 156.537657) (size 0.6) (drill 0.3) (layers "F.Cu" "B.Cu") (free yes) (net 3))
 (via (at 108.727527 156.537657) (size 0.6) (drill 0.3) (layers "F.Cu" "B.Cu") (free yes) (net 3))
 (via (at 104.227527 156.537657) (size 0.6) (drill 0.3) (layers "F.Cu" "B.Cu") (free yes) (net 3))
 (via (at 107.227527 156.537657) (size 0.6) (drill 0.3) (layers "F.Cu" "B.Cu") (free yes) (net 3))
 (segment (start 96.502527 157.168656) (end 96.502527 155.662658) (width 0.2) (layer "F.Cu") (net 46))
 (segment (start 96.502527 155.662658) (end 96.377527 155.537658) (width 0.2) (layer "F.Cu") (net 46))
 (segment (start 96.377527 155.537658) (end 96.377527 155.192657) (width 0.2) (layer "F.Cu") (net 46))
 (segment (start 96.477527 157.193656) (end 96.502527 157.168656) (width 0.2) (layer "F.Cu") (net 46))
 (segment (start 96.477527 158.468657) (end 96.477527 157.193656) (width 0.2) (layer "F.Cu") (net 46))
 (segment (start 97.077527 155.537658) (end 97.077527 155.192657) (width 0.2) (layer "F.Cu") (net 44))
 (segment (start 96.977527 158.468657) (end 96.977527 157.193656) (width 0.2) (layer "F.Cu") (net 44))
 (segment (start 96.952527 157.168656) (end 96.952527 155.662658) (width 0.2) (layer "F.Cu") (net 44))
 (segment (start 96.952527 155.662658) (end 97.077527 155.537658) (width 0.2) (layer "F.Cu") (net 44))
 (segment (start 96.977527 157.193656) (end 96.952527 157.168656) (width 0.2) (layer "F.Cu") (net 44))
 (segment (start 102.477527 157.193656) (end 102.502527 157.168656) (width 0.2) (layer "F.Cu") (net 1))
 (segment (start 102.502527 157.168656) (end 102.502527 155.662658) (width 0.2) (layer "F.Cu") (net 1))
 (segment (start 102.377527 155.537658) (end 102.377527 155.192657) (width 0.2) (layer "F.Cu") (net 1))
 (segment (start 102.477527 158.468657) (end 102.477527 157.193656) (width 0.2) (layer "F.Cu") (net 1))
 (segment (start 102.502527 155.662658) (end 102.377527 155.537658) (width 0.2) (layer "F.Cu") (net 1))
 (segment (start 102.952527 155.662658) (end 103.077527 155.537658) (width 0.2) (layer "F.Cu") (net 25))
 (segment (start 102.952527 157.168656) (end 102.952527 155.662658) (width 0.2) (layer "F.Cu") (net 25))
 (segment (start 102.977527 158.468657) (end 102.977527 157.193656) (width 0.2) (layer "F.Cu") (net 25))
 (segment (start 103.077527 155.537658) (end 103.077527 155.192657) (width 0.2) (layer "F.Cu") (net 25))
 (segment (start 102.977527 157.193656) (end 102.952527 157.168656) (width 0.2) (layer "F.Cu") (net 25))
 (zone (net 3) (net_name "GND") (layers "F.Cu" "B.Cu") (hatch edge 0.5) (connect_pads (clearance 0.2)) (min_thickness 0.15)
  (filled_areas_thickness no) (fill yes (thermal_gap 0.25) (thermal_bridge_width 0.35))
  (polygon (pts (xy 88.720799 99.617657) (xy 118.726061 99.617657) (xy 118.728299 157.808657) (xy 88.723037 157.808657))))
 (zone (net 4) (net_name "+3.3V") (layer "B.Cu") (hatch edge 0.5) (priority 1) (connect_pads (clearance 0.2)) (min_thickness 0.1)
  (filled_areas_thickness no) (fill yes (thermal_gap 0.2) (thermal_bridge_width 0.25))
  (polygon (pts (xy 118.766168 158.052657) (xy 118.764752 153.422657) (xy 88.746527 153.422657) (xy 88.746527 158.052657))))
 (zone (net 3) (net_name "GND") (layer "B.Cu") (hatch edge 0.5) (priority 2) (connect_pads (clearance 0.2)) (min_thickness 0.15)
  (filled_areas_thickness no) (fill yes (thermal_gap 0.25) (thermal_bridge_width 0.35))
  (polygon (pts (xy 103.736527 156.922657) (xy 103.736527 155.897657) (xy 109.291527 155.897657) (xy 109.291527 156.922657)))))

